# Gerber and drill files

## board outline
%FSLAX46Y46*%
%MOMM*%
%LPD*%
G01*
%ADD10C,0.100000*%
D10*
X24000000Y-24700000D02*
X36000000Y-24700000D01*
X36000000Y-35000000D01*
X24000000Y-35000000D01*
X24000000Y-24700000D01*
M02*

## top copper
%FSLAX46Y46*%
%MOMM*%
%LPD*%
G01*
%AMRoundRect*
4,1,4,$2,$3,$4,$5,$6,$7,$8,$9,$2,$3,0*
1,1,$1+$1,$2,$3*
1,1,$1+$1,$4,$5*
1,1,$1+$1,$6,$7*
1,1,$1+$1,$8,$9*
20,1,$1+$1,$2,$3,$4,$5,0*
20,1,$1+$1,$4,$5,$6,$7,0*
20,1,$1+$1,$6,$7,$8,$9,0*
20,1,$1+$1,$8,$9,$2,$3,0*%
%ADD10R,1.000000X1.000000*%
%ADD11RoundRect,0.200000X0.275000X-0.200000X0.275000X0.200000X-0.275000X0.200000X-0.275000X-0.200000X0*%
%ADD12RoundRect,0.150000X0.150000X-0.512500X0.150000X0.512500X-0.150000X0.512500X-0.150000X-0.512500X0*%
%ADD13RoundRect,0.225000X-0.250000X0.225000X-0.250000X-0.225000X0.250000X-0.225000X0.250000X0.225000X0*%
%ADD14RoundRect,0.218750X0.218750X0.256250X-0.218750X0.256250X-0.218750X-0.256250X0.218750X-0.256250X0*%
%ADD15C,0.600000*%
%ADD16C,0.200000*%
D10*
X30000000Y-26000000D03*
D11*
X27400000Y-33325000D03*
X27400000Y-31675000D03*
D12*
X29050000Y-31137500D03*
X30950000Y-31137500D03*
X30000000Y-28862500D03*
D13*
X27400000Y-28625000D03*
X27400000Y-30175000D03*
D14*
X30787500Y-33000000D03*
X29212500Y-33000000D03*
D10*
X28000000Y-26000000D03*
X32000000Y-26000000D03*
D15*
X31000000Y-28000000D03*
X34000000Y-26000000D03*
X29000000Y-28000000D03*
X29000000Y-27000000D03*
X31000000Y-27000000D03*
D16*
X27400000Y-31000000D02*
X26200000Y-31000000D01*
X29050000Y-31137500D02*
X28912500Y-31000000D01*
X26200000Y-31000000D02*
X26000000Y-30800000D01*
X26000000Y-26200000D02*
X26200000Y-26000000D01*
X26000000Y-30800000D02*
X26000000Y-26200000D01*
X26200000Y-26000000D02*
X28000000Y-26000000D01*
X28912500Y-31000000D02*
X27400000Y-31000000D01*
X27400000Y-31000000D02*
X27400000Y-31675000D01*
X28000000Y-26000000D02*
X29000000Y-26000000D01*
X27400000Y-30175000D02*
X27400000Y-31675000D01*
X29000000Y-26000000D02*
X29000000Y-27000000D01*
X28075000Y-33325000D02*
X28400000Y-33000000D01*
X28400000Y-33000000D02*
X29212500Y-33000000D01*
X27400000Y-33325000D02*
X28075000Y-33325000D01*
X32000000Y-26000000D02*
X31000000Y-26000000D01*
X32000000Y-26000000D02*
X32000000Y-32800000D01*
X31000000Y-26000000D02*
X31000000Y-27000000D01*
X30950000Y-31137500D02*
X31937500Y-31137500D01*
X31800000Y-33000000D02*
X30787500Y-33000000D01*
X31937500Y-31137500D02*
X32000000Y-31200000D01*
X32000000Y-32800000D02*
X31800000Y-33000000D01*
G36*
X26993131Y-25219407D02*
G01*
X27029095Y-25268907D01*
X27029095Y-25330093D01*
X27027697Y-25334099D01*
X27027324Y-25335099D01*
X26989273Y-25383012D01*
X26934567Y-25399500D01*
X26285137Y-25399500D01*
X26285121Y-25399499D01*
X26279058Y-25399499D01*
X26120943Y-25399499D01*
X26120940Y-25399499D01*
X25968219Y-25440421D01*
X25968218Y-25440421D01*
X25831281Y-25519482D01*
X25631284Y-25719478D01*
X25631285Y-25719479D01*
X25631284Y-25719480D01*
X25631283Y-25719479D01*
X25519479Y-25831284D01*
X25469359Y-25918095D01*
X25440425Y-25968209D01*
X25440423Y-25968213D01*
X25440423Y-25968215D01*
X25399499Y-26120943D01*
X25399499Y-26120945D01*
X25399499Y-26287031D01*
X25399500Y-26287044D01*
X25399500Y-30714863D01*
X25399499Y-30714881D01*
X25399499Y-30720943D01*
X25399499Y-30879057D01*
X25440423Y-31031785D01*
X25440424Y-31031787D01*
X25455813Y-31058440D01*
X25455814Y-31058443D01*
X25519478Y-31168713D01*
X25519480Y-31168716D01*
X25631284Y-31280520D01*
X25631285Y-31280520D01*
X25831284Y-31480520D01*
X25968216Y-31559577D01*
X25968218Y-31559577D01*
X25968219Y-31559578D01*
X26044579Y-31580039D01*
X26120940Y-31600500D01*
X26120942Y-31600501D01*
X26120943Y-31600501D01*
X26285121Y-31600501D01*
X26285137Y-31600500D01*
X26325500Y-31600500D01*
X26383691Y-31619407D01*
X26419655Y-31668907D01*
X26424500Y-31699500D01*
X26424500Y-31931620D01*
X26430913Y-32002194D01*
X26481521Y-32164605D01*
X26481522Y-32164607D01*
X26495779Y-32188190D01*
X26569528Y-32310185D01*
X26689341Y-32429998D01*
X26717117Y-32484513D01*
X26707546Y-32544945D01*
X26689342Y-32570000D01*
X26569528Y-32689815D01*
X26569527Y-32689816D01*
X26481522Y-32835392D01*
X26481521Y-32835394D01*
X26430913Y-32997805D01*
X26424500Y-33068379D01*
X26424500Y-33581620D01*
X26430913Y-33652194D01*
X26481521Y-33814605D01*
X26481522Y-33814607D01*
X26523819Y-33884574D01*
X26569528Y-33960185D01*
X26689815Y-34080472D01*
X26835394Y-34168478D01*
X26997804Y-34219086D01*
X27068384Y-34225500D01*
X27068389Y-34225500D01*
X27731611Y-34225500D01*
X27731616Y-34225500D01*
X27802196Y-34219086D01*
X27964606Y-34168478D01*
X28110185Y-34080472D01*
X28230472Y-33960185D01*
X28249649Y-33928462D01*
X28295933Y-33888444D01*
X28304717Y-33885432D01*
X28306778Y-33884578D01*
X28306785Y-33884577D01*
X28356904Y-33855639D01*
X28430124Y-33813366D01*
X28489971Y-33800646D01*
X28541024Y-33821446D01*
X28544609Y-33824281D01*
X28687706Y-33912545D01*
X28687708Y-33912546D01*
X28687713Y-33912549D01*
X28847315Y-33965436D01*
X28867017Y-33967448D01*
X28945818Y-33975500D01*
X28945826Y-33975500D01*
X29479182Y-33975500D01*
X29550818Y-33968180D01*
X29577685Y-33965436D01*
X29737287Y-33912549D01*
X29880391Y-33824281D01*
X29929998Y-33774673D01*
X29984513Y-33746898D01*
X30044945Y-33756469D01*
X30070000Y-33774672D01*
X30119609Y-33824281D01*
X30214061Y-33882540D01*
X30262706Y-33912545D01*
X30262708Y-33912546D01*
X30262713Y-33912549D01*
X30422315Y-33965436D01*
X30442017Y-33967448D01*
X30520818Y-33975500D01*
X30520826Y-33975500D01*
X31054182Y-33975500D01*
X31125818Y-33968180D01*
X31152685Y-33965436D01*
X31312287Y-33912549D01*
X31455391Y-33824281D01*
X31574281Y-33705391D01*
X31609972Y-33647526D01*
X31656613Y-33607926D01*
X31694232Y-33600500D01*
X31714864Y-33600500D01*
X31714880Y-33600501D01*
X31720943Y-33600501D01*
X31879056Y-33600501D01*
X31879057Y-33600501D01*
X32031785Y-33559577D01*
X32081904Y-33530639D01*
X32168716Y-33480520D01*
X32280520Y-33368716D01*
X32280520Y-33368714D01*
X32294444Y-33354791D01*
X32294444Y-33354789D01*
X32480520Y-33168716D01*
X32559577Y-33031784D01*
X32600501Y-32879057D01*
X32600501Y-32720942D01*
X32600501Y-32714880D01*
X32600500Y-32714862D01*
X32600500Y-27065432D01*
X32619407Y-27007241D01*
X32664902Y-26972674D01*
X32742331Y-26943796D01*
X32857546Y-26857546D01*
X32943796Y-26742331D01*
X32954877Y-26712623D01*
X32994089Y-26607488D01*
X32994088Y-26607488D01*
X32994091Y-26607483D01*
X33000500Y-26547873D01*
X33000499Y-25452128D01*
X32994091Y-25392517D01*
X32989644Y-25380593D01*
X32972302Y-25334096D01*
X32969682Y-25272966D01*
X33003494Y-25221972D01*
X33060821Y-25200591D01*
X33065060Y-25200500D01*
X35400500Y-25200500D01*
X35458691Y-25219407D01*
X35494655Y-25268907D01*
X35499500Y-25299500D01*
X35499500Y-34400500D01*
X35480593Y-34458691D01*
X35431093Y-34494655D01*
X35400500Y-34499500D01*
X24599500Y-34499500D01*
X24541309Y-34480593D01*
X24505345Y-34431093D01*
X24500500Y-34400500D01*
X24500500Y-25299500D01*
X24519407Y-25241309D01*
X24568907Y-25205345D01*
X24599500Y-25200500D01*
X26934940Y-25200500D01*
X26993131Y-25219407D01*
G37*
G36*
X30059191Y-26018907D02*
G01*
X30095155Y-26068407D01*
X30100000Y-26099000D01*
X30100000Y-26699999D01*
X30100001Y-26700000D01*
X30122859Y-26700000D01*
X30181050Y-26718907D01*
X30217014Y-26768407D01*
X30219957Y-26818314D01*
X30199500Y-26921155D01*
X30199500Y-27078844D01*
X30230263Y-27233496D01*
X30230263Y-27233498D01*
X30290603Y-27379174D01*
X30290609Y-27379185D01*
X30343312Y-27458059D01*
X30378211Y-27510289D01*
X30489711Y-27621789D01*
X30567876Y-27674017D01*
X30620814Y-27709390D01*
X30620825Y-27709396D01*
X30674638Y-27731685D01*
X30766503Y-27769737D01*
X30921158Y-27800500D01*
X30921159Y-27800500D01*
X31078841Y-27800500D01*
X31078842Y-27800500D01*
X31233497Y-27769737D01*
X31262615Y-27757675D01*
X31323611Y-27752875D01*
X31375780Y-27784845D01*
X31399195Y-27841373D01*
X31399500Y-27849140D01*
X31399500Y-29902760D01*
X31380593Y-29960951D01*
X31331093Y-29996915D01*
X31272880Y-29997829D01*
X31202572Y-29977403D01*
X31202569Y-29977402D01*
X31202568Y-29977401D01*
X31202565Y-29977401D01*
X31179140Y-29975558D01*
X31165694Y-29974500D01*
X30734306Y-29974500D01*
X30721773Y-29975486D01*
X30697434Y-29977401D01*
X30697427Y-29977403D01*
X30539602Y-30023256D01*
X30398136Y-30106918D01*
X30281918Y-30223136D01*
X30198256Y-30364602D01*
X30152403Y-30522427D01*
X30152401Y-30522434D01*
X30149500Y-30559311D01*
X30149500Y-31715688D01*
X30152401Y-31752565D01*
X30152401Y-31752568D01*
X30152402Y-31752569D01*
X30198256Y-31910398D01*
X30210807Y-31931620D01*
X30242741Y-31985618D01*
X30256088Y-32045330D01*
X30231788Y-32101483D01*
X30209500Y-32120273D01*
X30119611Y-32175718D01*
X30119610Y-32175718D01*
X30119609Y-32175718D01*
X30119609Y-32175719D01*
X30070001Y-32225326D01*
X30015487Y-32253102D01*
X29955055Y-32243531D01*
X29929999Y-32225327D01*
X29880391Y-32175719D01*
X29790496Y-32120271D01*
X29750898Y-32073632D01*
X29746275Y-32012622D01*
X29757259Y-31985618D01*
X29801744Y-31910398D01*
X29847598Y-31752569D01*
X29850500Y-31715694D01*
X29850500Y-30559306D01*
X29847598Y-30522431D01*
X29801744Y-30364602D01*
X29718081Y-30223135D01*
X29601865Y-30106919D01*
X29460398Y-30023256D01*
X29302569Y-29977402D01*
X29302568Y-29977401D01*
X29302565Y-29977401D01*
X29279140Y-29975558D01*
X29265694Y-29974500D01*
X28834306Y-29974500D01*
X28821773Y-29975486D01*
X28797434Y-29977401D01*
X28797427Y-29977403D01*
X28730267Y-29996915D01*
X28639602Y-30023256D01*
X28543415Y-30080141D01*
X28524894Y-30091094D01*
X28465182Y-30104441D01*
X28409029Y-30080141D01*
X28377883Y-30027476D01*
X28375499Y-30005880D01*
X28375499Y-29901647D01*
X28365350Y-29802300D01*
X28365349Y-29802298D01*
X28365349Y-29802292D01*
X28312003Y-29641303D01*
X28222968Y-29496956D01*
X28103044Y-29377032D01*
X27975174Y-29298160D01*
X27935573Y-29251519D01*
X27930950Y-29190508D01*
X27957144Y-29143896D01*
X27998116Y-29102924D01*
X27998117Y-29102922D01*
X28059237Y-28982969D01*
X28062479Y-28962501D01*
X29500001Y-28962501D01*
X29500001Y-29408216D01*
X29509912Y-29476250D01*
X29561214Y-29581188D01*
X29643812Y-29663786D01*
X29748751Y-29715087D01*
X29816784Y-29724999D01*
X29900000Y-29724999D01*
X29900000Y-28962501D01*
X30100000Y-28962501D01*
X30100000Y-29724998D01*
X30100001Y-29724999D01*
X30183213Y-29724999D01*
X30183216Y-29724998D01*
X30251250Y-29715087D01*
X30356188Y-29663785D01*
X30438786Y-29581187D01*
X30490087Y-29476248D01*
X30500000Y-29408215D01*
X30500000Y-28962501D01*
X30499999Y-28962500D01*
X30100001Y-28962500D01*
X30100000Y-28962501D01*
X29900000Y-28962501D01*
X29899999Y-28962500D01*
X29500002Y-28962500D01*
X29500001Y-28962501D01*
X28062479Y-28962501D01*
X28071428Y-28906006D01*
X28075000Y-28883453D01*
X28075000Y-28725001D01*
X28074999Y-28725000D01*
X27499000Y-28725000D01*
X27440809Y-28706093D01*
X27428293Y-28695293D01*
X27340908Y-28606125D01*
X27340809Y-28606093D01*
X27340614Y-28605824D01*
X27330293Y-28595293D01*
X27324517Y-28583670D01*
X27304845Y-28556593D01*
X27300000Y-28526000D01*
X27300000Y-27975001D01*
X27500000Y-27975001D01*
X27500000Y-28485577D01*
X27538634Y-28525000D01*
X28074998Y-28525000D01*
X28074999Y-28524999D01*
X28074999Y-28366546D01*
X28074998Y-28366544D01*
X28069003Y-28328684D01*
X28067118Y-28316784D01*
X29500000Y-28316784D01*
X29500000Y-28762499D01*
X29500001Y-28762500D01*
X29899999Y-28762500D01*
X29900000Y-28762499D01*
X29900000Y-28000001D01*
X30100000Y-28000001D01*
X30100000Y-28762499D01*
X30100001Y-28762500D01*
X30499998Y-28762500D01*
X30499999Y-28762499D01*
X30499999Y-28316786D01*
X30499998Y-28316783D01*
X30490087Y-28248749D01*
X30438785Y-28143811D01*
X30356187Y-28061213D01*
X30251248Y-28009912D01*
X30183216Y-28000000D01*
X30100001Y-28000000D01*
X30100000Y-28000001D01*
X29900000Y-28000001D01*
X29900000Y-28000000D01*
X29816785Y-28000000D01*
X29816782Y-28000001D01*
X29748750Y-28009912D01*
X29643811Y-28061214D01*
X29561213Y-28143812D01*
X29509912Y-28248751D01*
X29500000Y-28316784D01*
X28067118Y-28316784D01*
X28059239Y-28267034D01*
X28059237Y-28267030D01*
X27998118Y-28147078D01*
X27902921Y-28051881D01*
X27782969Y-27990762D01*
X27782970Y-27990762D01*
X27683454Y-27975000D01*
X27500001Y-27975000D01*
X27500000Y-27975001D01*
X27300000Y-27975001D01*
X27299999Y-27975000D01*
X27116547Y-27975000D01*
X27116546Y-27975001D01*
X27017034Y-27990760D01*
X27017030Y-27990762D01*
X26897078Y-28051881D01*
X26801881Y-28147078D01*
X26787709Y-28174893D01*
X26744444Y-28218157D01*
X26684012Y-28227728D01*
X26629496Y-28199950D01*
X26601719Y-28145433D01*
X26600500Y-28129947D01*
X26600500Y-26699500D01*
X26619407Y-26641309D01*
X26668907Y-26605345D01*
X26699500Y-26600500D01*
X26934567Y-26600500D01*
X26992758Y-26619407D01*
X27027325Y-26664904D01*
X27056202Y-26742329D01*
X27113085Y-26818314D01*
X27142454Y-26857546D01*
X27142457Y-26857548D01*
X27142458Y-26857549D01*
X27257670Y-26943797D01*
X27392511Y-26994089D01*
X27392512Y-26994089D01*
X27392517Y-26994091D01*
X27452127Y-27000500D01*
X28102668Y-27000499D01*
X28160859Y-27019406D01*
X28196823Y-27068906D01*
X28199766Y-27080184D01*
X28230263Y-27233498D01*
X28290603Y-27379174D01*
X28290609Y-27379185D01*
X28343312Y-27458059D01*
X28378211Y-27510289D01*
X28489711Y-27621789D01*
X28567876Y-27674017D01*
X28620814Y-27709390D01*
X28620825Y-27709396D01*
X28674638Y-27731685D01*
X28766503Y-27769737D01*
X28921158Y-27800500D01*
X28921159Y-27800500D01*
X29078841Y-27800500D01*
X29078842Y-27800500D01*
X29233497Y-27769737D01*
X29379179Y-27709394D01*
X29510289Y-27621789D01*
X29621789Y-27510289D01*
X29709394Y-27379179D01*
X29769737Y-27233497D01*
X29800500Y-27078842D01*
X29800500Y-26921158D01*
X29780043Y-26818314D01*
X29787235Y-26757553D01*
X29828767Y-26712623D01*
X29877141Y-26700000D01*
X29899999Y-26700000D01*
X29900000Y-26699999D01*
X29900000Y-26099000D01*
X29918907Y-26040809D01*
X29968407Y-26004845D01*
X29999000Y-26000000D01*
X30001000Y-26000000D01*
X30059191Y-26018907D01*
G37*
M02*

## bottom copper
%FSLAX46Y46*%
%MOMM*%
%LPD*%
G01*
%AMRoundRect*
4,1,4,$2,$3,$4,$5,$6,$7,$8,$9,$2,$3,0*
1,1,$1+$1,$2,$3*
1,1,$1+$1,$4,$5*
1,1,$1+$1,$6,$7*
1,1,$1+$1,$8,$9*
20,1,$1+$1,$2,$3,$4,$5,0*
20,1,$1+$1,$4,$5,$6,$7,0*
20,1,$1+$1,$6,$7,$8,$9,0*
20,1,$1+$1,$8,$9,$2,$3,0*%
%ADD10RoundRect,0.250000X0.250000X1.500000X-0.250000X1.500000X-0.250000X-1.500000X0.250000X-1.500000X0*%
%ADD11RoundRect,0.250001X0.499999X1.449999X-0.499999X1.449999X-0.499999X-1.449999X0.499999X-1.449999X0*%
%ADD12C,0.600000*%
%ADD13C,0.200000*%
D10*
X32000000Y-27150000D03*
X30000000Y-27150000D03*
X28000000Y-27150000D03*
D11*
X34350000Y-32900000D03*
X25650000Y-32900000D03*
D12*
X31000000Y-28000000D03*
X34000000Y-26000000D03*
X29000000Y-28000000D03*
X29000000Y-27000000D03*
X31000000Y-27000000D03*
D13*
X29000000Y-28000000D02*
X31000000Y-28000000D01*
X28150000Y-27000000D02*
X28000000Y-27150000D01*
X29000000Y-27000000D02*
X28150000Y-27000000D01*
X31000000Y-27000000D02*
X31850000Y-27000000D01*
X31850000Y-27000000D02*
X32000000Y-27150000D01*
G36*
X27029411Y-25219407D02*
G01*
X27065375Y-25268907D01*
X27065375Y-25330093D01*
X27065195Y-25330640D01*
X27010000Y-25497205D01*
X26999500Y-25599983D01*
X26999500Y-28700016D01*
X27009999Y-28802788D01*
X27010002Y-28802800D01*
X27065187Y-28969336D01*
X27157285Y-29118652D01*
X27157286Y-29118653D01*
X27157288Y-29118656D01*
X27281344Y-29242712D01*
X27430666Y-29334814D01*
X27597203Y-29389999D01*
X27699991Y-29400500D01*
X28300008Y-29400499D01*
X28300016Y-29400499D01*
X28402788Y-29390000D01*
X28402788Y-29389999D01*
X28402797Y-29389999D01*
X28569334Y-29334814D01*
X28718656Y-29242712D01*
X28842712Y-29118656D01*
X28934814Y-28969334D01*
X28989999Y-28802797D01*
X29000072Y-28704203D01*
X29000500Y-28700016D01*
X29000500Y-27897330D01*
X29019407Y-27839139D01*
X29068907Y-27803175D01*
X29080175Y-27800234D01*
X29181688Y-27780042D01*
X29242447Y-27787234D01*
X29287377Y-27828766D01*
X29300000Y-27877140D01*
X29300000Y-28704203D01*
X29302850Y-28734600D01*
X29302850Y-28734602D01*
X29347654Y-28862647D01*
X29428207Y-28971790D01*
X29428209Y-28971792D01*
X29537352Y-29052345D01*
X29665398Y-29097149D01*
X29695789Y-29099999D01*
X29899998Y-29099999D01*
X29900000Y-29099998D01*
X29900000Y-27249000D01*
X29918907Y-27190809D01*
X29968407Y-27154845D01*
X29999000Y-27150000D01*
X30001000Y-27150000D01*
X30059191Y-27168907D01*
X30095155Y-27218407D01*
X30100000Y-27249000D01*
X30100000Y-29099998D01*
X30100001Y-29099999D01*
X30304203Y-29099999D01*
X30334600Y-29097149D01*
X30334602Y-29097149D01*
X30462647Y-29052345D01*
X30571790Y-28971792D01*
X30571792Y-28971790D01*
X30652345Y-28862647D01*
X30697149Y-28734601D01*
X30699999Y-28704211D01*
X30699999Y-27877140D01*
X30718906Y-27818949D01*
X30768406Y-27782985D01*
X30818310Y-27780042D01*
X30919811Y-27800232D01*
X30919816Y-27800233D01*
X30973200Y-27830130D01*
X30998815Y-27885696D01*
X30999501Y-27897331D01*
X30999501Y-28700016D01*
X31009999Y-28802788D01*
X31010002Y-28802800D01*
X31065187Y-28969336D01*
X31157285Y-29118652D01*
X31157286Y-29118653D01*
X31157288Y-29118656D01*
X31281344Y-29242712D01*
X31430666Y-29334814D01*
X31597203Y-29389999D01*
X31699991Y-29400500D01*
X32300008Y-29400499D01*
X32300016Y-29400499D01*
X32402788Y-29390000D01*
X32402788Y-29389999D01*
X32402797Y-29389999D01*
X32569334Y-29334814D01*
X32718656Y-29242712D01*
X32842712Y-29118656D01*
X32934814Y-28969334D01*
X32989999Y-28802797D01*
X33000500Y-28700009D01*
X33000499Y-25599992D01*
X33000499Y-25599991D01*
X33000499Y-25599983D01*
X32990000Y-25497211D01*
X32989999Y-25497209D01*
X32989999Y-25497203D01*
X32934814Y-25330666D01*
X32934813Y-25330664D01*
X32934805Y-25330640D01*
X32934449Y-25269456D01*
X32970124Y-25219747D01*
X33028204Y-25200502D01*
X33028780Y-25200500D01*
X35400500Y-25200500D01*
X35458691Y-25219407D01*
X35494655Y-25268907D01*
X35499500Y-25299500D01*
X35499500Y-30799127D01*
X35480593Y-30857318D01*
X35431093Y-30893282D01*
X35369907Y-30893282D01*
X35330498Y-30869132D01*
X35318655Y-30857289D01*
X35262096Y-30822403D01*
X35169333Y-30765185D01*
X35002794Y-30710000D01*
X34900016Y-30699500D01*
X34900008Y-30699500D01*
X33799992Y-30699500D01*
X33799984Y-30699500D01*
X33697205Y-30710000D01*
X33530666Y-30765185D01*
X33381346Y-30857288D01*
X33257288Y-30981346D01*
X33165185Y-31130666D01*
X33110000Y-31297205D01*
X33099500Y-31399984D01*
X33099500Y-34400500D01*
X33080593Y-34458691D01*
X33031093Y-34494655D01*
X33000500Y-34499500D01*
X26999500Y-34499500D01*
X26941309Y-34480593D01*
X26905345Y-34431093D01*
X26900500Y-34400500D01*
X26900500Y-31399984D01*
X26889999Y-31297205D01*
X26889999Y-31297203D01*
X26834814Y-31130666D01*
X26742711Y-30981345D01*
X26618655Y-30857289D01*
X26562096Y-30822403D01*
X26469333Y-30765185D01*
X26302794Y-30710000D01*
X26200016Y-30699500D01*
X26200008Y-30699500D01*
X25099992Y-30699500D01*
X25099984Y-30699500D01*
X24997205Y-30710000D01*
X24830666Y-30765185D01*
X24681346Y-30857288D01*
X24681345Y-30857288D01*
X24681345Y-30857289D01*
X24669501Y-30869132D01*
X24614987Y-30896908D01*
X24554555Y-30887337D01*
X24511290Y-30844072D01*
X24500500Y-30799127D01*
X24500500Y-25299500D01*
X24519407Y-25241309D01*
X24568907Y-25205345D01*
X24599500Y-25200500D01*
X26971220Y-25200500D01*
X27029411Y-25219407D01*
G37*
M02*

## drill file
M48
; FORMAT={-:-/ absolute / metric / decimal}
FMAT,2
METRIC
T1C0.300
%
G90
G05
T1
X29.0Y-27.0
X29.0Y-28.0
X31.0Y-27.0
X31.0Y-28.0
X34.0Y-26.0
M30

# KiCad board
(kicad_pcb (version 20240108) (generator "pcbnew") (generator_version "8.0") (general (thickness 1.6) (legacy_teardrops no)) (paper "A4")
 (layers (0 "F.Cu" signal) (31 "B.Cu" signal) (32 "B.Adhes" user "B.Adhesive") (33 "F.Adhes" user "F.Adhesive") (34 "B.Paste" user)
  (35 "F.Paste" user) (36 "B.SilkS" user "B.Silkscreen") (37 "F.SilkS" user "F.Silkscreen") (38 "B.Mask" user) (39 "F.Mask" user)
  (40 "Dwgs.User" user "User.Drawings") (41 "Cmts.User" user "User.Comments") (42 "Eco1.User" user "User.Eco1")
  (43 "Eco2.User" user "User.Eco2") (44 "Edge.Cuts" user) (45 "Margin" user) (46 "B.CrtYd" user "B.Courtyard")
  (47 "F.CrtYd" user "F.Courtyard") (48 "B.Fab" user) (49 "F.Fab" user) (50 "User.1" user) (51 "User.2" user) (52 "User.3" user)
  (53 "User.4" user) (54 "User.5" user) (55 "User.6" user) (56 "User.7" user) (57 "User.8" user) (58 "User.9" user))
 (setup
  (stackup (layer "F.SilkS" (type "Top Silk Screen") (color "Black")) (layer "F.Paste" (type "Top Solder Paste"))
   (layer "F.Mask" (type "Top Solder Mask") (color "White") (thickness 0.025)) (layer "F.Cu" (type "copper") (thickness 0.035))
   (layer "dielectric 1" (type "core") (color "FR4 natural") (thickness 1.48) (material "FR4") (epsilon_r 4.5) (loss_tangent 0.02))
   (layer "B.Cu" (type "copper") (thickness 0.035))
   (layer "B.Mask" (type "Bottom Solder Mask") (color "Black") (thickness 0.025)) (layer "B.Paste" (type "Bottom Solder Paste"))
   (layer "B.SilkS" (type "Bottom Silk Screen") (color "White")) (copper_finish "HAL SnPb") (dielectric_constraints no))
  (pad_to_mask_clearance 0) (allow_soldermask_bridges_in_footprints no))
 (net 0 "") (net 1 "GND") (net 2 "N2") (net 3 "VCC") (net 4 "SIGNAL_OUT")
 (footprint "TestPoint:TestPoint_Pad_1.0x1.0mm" (layer "F.Cu") (at 30 26 90)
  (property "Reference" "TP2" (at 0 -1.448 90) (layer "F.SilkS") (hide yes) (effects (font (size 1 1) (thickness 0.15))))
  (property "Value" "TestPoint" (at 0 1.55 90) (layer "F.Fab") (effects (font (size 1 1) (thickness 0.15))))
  (pad "1" smd rect (at 0 0 90) (size 1 1) (layers "F.Cu" "F.Mask") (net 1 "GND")))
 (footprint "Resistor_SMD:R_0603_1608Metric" (layer "F.Cu") (at 27.4 32.5 90)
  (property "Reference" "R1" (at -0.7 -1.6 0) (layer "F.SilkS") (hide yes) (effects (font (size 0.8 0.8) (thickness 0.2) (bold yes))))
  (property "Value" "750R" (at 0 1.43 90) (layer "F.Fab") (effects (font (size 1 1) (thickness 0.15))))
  (pad "1" smd roundrect (at -0.825 0 90) (size 0.8 0.95) (layers "F.Cu" "F.Paste" "F.Mask") (roundrect_rratio 0.25) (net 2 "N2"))
  (pad "2" smd roundrect (at 0.825 0 90) (size 0.8 0.95) (layers "F.Cu" "F.Paste" "F.Mask") (roundrect_rratio 0.25) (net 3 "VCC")))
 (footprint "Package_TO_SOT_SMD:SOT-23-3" (layer "F.Cu") (at 30 30 90)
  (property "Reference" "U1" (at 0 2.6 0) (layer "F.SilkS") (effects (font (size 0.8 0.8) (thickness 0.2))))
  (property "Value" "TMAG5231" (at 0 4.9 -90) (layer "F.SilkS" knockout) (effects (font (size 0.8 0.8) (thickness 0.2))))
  (pad "1" smd roundrect (at -1.1375 -0.95 90) (size 1.325 0.6) (layers "F.Cu" "F.Paste" "F.Mask") (roundrect_rratio 0.25) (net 3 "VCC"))
  (pad "2" smd roundrect (at -1.1375 0.95 90) (size 1.325 0.6) (layers "F.Cu" "F.Paste" "F.Mask") (roundrect_rratio 0.25)
   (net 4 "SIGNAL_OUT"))
  (pad "3" smd roundrect (at 1.1375 0 90) (size 1.325 0.6) (layers "F.Cu" "F.Paste" "F.Mask") (roundrect_rratio 0.25) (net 1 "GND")))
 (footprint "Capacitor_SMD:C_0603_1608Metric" (layer "F.Cu") (at 27.4 29.4 -90)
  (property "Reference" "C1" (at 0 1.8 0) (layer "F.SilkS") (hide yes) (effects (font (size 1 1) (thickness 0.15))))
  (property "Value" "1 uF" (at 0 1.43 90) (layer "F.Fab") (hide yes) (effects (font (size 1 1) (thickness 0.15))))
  (pad "1" smd roundrect (at -0.775 0 270) (size 0.9 0.95) (layers "F.Cu" "F.Paste" "F.Mask") (roundrect_rratio 0.25) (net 1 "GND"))
  (pad "2" smd roundrect (at 0.775 0 270) (size 0.9 0.95) (layers "F.Cu" "F.Paste" "F.Mask") (roundrect_rratio 0.25) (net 3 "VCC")))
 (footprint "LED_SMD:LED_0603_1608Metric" (layer "F.Cu") (at 30 33 180)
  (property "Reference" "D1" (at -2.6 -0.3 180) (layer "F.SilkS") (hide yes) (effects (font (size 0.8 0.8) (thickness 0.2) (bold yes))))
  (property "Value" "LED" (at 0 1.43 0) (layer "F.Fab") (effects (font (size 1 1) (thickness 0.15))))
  (pad "1" smd roundrect (at -0.7875 0 180) (size 0.875 0.95) (layers "F.Cu" "F.Paste" "F.Mask") (roundrect_rratio 0.25)
   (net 4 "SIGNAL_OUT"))
  (pad "2" smd roundrect (at 0.7875 0 180) (size 0.875 0.95) (layers "F.Cu" "F.Paste" "F.Mask") (roundrect_rratio 0.25) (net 2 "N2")))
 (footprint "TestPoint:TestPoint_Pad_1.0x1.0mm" (layer "F.Cu") (at 28 26 90)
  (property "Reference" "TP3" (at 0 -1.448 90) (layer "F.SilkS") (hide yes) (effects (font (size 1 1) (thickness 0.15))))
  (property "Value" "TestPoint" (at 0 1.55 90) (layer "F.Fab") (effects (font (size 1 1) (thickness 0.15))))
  (pad "1" smd rect (at 0 0 90) (size 1 1) (layers "F.Cu" "F.Mask") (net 3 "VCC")))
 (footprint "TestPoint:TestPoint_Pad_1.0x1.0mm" (layer "F.Cu") (at 32 26)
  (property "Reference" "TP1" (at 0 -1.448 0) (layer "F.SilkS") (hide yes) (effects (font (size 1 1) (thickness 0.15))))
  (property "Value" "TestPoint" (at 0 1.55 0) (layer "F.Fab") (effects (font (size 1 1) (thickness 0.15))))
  (pad "1" smd rect (at 0 0) (size 1 1) (layers "F.Cu" "F.Mask") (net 4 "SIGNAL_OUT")))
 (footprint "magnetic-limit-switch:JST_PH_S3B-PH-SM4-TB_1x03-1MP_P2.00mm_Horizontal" (layer "B.Cu") (at 30 30 180)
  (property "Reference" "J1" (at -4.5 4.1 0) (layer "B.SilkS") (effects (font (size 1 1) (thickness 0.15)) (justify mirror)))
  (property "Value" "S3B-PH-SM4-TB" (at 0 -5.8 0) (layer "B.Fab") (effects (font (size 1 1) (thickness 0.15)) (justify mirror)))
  (pad "1" smd roundrect (at -2 2.85 180) (size 1 3.5) (layers "B.Cu" "B.Paste" "B.Mask") (roundrect_rratio 0.25) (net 4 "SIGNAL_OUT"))
  (pad "2" smd roundrect (at 0 2.85 180) (size 1 3.5) (layers "B.Cu" "B.Paste" "B.Mask") (roundrect_rratio 0.25) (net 1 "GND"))
  (pad "3" smd roundrect (at 2 2.85 180) (size 1 3.5) (layers "B.Cu" "B.Paste" "B.Mask") (roundrect_rratio 0.25) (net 3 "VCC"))
  (pad "MP" smd roundrect (at -4.35 -2.9 180) (size 1.5 3.4) (layers "B.Cu" "B.Paste" "B.Mask") (roundrect_rratio 0.166667))
  (pad "MP" smd roundrect (at 4.35 -2.9 180) (size 1.5 3.4) (layers "B.Cu" "B.Paste" "B.Mask") (roundrect_rratio 0.166667)))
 (gr_rect (start 24 24.7) (end 36 35) (stroke (width 0.1) (type default)) (fill none) (layer "Edge.Cuts"))
 (via (at 31 28) (size 0.6) (drill 0.3) (layers "F.Cu" "B.Cu") (free yes) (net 1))
 (via (at 34 26) (size 0.6) (drill 0.3) (layers "F.Cu" "B.Cu") (free yes) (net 1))
 (via (at 29 28) (size 0.6) (drill 0.3) (layers "F.Cu" "B.Cu") (free yes) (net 1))
 (segment (start 29 28) (end 31 28) (width 0.2) (layer "B.Cu") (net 1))
 (segment (start 27.4 31) (end 26.2 31) (width 0.2) (layer "F.Cu") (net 3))
 (segment (start 29.05 31.1375) (end 28.9125 31) (width 0.2) (layer "F.Cu") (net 3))
 (segment (start 26.2 31) (end 26 30.8) (width 0.2) (layer "F.Cu") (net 3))
 (segment (start 26 26.2) (end 26.2 26) (width 0.2) (layer "F.Cu") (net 3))
 (segment (start 26 30.8) (end 26 26.2) (width 0.2) (layer "F.Cu") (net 3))
 (segment (start 26.2 26) (end 28 26) (width 0.2) (layer "F.Cu") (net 3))
 (segment (start 28.9125 31) (end 27.4 31) (width 0.2) (layer "F.Cu") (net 3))
 (segment (start 27.4 31) (end 27.4 31.675) (width 0.2) (layer "F.Cu") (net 3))
 (segment (start 28 26) (end 29 26) (width 0.2) (layer "F.Cu") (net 3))
 (segment (start 27.4 30.175) (end 27.4 31.675) (width 0.2) (layer "F.Cu") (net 3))
 (segment (start 29 26) (end 29 27) (width 0.2) (layer "F.Cu") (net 3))
 (via (at 29 27) (size 0.6) (drill 0.3) (layers "F.Cu" "B.Cu") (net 3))
 (segment (start 28.15 27) (end 28 27.15) (width 0.2) (layer "B.Cu") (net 3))
 (segment (start 29 27) (end 28.15 27) (width 0.2) (layer "B.Cu") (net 3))
 (segment (start 28.075 33.325) (end 28.4 33) (width 0.2) (layer "F.Cu") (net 2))
 (segment (start 28.4 33) (end 29.2125 33) (width 0.2) (layer "F.Cu") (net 2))
 (segment (start 27.4 33.325) (end 28.075 33.325) (width 0.2) (layer "F.Cu") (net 2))
 (segment (start 32 26) (end 31 26) (width 0.2) (layer "F.Cu") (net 4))
 (segment (start 32 26) (end 32 32.8) (width 0.2) (layer "F.Cu") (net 4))
 (segment (start 31 26) (end 31 27) (width 0.2) (layer "F.Cu") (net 4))
 (segment (start 30.95 31.1375) (end 31.9375 31.1375) (width 0.2) (layer "F.Cu") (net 4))
 (segment (start 31.8 33) (end 30.7875 33) (width 0.2) (layer "F.Cu") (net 4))
 (segment (start 31.9375 31.1375) (end 32 31.2) (width 0.2) (layer "F.Cu") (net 4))
 (segment (start 32 32.8) (end 31.8 33) (width 0.2) (layer "F.Cu") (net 4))
 (via (at 31 27) (size 0.6) (drill 0.3) (layers "F.Cu" "B.Cu") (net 4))
 (segment (start 31 27) (end 31.85 27) (width 0.2) (layer "B.Cu") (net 4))
 (segment (start 31.85 27) (end 32 27.15) (width 0.2) (layer "B.Cu") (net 4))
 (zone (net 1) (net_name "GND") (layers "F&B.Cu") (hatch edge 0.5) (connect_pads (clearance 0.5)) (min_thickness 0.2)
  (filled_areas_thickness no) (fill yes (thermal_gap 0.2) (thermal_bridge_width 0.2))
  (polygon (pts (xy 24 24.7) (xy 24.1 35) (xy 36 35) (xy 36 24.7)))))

